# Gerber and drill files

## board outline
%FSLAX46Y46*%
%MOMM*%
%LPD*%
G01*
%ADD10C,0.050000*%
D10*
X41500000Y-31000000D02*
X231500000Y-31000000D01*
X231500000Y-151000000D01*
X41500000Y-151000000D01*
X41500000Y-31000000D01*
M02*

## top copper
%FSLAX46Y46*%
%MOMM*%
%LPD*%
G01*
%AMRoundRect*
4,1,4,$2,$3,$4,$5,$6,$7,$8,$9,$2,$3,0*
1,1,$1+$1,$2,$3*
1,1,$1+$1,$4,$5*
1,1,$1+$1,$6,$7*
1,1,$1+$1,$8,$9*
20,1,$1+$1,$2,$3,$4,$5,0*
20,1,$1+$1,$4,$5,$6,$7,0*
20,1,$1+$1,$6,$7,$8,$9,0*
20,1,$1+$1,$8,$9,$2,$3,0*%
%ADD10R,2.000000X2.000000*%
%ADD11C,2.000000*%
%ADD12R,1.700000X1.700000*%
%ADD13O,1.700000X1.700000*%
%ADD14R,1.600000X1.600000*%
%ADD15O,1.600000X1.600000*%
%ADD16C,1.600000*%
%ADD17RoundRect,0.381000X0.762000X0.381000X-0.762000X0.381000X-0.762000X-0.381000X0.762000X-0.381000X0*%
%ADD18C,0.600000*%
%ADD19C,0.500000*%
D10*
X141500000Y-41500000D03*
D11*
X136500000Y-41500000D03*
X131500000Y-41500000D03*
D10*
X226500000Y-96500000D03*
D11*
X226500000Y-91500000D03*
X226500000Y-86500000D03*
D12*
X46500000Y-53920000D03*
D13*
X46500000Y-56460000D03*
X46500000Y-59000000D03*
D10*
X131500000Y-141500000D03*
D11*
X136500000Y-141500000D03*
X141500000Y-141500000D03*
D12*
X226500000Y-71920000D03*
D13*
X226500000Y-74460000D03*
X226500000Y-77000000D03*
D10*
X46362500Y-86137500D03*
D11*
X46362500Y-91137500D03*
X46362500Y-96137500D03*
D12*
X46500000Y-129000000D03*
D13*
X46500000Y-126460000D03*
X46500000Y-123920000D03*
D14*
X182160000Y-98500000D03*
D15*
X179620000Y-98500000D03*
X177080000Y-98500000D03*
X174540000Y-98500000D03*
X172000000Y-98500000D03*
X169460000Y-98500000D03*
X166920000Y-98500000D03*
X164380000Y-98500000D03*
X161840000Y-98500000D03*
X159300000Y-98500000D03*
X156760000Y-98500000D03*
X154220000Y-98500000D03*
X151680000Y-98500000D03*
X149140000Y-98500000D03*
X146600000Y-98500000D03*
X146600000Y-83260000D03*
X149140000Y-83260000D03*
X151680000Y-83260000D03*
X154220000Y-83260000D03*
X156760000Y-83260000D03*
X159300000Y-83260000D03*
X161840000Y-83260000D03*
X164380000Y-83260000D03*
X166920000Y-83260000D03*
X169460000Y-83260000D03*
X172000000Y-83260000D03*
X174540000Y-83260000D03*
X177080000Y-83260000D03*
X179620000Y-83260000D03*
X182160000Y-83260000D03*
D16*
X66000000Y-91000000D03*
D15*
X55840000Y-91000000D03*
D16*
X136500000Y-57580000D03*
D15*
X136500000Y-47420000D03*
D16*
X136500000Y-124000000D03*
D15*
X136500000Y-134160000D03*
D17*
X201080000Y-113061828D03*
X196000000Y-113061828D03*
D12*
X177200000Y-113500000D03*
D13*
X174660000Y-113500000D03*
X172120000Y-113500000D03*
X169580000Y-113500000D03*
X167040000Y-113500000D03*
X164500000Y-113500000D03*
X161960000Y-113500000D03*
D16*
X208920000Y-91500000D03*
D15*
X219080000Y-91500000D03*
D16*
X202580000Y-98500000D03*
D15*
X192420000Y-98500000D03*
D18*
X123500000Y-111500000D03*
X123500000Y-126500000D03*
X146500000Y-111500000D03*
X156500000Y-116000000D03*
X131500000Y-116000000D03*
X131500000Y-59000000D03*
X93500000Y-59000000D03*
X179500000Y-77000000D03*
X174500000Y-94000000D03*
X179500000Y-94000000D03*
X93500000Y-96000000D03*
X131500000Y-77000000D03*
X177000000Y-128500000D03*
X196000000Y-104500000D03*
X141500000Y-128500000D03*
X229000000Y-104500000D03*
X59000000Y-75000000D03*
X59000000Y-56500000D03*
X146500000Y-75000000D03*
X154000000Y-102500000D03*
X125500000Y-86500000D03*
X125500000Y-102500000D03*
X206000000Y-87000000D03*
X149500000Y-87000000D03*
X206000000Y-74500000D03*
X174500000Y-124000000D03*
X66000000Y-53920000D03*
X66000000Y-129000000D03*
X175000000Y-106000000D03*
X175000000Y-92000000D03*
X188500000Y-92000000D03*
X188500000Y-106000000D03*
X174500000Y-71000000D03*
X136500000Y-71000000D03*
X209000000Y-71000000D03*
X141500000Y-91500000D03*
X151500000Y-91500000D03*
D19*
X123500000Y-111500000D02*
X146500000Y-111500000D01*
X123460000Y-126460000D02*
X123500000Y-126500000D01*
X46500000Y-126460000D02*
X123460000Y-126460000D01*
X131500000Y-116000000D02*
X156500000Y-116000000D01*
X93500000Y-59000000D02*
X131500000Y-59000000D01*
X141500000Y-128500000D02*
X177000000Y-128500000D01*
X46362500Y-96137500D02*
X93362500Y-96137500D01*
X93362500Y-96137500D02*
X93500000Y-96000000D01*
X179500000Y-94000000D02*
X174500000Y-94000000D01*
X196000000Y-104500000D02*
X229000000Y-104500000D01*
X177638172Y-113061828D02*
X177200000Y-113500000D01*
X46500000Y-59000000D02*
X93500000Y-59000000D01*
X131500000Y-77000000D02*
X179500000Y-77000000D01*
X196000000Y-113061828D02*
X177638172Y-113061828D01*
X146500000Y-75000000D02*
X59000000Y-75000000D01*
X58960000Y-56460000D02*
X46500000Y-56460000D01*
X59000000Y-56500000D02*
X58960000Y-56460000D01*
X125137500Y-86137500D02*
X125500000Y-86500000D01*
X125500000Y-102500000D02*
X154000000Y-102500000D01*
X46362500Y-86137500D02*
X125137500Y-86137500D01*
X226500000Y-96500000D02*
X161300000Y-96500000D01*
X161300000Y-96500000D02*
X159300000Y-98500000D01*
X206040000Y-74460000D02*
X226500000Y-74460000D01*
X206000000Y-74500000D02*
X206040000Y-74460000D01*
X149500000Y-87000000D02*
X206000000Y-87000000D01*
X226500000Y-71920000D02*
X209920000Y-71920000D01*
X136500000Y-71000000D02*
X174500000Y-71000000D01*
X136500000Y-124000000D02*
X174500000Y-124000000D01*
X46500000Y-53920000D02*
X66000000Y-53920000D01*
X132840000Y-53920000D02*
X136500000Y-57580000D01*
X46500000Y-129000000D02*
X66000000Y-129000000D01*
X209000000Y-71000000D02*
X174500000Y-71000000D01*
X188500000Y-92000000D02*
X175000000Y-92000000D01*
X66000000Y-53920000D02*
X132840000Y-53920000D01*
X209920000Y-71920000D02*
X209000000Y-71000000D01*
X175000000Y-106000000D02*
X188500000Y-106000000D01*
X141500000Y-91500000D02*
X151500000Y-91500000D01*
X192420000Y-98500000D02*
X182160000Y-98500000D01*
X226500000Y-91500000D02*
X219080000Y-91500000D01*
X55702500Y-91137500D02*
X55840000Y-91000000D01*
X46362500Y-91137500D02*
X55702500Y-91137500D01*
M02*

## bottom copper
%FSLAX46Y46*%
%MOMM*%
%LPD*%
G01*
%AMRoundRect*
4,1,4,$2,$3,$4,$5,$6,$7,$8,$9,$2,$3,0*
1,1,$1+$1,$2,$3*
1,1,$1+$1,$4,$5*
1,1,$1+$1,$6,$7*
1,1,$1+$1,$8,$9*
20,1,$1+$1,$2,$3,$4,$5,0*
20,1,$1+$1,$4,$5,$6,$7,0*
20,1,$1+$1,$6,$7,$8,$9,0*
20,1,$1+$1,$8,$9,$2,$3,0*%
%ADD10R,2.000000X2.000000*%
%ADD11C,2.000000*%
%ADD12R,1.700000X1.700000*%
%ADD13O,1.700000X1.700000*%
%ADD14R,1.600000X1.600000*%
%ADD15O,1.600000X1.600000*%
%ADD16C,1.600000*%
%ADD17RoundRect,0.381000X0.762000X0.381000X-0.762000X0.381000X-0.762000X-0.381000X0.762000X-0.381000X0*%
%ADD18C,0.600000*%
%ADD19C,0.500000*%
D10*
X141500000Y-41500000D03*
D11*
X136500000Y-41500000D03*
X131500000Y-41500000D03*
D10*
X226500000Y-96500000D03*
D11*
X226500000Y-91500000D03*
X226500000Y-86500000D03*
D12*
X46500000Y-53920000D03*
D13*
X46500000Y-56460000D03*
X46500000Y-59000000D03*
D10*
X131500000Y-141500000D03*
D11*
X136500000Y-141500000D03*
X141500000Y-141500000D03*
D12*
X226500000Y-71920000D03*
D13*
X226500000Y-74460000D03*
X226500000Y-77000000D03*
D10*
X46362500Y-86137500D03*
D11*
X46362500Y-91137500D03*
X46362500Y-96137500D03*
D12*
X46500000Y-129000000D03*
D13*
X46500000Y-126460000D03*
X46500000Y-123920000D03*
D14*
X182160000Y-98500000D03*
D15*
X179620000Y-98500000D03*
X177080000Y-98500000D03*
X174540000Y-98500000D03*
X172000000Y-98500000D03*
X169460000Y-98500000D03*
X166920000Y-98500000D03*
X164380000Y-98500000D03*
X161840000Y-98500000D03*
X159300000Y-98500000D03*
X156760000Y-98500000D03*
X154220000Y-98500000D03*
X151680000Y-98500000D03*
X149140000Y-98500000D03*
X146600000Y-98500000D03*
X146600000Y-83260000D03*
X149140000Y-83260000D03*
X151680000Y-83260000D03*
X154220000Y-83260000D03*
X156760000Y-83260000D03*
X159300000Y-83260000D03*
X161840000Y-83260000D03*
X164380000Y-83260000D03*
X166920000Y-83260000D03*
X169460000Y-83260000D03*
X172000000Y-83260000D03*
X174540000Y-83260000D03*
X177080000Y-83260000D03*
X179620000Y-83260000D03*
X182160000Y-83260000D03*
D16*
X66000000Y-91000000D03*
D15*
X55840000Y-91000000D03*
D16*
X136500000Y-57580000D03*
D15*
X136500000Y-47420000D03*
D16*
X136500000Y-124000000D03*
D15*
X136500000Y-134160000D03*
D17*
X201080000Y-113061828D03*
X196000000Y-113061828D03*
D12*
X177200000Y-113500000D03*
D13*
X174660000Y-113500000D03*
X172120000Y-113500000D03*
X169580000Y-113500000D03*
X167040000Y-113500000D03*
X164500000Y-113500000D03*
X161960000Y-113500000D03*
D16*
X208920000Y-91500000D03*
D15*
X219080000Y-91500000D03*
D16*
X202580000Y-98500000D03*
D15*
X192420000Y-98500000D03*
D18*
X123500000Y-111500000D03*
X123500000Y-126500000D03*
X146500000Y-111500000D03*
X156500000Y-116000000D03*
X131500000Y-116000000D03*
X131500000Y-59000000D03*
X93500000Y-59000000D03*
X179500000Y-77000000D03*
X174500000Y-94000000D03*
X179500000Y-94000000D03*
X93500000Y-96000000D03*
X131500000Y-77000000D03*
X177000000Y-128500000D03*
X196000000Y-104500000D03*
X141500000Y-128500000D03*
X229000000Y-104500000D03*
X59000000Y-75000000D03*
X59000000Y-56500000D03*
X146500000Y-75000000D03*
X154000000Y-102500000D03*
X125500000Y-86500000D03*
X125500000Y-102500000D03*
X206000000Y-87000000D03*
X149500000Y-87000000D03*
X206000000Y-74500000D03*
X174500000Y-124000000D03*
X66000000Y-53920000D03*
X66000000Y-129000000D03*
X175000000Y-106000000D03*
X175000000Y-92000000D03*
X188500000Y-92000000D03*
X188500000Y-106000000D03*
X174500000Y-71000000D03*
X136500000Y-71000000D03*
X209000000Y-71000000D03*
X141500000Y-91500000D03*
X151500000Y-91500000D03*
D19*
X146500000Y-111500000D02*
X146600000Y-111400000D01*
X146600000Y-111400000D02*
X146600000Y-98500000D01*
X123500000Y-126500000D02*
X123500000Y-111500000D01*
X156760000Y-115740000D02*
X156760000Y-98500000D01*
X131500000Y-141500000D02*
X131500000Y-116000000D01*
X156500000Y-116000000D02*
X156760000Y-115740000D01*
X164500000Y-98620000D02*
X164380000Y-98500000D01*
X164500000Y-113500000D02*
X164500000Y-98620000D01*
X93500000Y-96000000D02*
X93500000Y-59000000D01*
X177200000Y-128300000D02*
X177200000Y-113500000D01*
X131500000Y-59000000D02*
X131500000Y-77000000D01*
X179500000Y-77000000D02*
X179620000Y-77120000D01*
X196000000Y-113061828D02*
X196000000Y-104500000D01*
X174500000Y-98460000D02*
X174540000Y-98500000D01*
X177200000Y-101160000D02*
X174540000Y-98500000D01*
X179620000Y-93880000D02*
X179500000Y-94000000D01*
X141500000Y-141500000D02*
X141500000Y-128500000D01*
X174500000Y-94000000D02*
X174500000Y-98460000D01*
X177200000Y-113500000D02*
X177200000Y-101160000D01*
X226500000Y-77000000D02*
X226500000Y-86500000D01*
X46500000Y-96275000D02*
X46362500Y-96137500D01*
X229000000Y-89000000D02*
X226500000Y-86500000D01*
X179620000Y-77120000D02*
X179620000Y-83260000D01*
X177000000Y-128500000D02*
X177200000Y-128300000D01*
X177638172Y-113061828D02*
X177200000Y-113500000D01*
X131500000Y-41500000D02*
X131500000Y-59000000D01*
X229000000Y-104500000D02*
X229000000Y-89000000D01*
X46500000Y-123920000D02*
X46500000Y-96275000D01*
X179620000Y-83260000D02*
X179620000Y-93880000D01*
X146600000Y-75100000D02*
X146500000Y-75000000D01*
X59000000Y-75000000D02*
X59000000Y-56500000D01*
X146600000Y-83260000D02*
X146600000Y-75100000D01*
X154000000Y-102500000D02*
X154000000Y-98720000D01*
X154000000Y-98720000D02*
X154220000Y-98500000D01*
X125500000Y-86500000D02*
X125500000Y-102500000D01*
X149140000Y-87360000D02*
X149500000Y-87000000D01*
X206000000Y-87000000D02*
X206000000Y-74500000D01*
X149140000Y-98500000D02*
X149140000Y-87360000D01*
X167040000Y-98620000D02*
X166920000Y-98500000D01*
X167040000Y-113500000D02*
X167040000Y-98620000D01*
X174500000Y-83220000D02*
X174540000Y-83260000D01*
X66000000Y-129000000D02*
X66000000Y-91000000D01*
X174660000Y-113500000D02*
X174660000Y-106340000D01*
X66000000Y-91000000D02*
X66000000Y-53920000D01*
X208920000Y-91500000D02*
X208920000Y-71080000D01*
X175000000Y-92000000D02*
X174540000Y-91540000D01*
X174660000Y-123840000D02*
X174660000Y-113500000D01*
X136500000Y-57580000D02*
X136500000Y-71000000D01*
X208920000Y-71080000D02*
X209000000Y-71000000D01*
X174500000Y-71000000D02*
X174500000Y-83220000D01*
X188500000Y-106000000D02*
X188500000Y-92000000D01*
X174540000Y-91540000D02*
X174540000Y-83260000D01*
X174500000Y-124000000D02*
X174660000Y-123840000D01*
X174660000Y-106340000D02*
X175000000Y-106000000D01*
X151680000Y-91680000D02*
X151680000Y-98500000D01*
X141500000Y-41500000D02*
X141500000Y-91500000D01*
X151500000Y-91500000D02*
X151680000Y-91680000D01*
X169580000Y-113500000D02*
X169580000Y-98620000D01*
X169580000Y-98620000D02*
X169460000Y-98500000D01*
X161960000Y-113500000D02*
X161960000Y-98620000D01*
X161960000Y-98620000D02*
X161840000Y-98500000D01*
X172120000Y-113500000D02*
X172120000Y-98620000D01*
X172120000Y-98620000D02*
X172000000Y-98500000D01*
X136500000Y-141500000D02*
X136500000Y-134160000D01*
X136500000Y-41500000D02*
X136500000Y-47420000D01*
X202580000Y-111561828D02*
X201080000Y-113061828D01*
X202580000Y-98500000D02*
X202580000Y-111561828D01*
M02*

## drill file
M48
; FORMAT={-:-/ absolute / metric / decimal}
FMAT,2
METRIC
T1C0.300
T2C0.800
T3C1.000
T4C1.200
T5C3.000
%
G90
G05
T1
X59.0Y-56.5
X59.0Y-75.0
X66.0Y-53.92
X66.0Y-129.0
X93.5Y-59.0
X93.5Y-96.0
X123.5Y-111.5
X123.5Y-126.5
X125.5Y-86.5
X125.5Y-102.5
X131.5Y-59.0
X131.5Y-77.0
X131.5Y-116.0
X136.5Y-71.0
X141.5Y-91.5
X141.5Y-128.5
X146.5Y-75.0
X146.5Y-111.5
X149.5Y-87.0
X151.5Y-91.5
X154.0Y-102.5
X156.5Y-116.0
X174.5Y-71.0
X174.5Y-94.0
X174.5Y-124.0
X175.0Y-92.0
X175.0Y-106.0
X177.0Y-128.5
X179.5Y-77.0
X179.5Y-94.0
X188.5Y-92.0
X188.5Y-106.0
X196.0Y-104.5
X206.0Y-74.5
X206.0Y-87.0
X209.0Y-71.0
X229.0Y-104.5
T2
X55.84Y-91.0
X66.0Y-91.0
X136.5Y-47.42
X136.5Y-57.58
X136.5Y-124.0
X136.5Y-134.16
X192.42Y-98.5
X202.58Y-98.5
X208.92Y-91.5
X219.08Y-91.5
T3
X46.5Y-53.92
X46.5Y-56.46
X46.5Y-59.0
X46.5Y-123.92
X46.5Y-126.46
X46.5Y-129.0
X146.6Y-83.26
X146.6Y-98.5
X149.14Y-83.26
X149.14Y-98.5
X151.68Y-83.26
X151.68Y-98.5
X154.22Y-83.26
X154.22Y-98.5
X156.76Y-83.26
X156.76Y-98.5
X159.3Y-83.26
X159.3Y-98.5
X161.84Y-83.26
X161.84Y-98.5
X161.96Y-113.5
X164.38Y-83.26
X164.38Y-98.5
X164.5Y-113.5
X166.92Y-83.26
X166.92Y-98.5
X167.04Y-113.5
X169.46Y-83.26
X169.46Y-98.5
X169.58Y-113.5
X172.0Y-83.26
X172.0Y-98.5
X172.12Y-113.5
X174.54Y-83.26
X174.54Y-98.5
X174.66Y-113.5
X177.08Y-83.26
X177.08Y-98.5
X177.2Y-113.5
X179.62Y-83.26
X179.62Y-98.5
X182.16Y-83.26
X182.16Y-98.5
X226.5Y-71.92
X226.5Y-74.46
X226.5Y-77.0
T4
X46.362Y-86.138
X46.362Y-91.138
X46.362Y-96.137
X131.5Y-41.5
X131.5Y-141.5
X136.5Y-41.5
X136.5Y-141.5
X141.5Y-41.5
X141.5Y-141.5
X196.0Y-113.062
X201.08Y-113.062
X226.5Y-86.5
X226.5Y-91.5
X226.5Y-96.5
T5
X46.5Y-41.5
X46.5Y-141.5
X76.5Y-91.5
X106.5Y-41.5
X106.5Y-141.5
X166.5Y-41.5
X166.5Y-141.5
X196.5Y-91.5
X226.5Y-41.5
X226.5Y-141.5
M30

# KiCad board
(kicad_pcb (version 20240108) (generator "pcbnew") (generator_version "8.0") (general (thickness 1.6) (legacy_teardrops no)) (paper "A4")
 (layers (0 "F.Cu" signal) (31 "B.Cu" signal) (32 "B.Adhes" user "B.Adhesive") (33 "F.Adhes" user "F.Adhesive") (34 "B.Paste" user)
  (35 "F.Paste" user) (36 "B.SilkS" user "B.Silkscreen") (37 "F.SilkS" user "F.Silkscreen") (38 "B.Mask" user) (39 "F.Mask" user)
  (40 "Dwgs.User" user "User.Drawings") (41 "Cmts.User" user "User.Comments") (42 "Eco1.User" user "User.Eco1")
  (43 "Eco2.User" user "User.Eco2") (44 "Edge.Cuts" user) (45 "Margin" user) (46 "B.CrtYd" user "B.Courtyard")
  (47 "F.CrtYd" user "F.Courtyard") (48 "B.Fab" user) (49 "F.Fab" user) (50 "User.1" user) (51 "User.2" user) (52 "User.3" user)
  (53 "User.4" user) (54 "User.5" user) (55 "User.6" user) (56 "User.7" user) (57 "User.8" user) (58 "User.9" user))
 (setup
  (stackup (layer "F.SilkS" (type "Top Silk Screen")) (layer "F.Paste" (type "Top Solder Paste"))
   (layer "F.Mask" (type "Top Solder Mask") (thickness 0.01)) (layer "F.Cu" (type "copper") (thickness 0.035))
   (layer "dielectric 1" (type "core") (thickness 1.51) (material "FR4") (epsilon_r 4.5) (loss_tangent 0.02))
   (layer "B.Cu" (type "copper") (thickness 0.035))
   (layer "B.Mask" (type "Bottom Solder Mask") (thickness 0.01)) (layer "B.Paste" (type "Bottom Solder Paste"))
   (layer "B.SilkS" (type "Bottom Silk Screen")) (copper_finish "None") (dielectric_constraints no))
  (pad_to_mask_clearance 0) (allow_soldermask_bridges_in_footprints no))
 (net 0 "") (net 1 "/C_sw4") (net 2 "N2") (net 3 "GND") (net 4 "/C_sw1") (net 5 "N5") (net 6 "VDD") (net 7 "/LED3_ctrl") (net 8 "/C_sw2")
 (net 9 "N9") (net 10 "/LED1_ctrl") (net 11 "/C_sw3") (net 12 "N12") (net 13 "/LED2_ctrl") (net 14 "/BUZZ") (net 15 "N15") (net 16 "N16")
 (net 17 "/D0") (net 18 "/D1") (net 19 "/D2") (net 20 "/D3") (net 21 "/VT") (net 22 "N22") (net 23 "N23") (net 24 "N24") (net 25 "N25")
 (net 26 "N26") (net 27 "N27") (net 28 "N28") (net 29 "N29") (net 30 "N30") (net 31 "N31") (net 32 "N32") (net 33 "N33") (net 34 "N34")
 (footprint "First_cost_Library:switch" (layer "F.Cu") (at 128.5 36.5 -90)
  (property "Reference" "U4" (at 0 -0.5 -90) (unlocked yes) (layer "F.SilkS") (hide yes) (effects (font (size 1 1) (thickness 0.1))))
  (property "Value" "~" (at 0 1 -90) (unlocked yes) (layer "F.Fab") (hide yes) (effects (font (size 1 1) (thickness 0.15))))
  (pad "1" thru_hole rect (at 5 -13 270) (size 2 2) (drill 1.2) (layers "*.Cu" "*.Mask") (remove_unused_layers no) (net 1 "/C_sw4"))
  (pad "2" thru_hole circle (at 5 -8 270) (size 2 2) (drill 1.2) (layers "*.Cu" "*.Mask") (remove_unused_layers no) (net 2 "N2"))
  (pad "3" thru_hole circle (at 5 -3 270) (size 2 2) (drill 1.2) (layers "*.Cu" "*.Mask") (remove_unused_layers no) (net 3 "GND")))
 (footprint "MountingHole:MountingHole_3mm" (layer "F.Cu") (at 196.5 91.5)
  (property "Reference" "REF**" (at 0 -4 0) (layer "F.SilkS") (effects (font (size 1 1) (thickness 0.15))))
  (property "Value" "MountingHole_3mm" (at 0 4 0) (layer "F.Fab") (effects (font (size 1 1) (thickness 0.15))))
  (pad "" np_thru_hole circle (at 0 0) (size 3 3) (drill 3) (layers "*.Cu" "*.Mask")))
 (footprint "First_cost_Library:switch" (layer "F.Cu") (at 231.5 83.5 180)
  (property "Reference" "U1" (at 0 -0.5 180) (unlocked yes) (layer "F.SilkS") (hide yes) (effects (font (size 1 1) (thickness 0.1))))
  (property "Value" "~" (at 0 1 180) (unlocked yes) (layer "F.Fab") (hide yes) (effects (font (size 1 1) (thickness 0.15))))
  (pad "1" thru_hole rect (at 5 -13 180) (size 2 2) (drill 1.2) (layers "*.Cu" "*.Mask") (remove_unused_layers no) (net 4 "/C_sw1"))
  (pad "2" thru_hole circle (at 5 -8 180) (size 2 2) (drill 1.2) (layers "*.Cu" "*.Mask") (remove_unused_layers no) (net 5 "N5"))
  (pad "3" thru_hole circle (at 5 -3 180) (size 2 2) (drill 1.2) (layers "*.Cu" "*.Mask") (remove_unused_layers no) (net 3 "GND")))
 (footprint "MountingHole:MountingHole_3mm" (layer "F.Cu") (at 76.5 91.5)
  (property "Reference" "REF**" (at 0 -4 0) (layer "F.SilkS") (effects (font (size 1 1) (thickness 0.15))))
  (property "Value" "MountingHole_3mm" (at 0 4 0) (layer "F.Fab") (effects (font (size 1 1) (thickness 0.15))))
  (pad "" np_thru_hole circle (at 0 0) (size 3 3) (drill 3) (layers "*.Cu" "*.Mask")))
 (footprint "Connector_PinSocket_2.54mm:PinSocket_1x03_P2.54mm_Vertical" (layer "F.Cu") (at 46.5 53.92)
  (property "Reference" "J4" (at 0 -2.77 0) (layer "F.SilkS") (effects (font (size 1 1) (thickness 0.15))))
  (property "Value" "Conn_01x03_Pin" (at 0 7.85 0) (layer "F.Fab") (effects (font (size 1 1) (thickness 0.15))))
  (pad "1" thru_hole rect (at 0 0) (size 1.7 1.7) (drill 1) (layers "*.Cu" "*.Mask") (remove_unused_layers no) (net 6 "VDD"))
  (pad "2" thru_hole oval (at 0 2.54) (size 1.7 1.7) (drill 1) (layers "*.Cu" "*.Mask") (remove_unused_layers no) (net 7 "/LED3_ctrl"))
  (pad "3" thru_hole oval (at 0 5.08) (size 1.7 1.7) (drill 1) (layers "*.Cu" "*.Mask") (remove_unused_layers no) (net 3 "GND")))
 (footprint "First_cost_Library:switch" (layer "F.Cu") (at 144.5 146.5 90)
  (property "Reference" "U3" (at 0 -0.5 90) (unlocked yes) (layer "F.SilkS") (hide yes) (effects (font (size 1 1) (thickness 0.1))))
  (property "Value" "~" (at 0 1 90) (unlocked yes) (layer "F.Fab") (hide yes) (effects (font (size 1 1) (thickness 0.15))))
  (pad "1" thru_hole rect (at 5 -13 90) (size 2 2) (drill 1.2) (layers "*.Cu" "*.Mask") (remove_unused_layers no) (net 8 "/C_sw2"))
  (pad "2" thru_hole circle (at 5 -8 90) (size 2 2) (drill 1.2) (layers "*.Cu" "*.Mask") (remove_unused_layers no) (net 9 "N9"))
  (pad "3" thru_hole circle (at 5 -3 90) (size 2 2) (drill 1.2) (layers "*.Cu" "*.Mask") (remove_unused_layers no) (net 3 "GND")))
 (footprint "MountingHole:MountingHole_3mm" (layer "F.Cu") (at 166.5 141.5)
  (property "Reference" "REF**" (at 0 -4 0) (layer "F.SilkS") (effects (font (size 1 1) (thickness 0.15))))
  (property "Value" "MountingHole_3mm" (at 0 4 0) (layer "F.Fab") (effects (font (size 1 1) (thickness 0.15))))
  (pad "" np_thru_hole circle (at 0 0) (size 3 3) (drill 3) (layers "*.Cu" "*.Mask")))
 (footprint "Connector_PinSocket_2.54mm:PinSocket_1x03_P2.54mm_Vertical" (layer "F.Cu") (at 226.5 71.92)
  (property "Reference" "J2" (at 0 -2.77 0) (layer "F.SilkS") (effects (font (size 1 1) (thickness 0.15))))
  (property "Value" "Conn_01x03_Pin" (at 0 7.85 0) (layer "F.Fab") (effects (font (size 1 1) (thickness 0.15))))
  (pad "1" thru_hole rect (at 0 0) (size 1.7 1.7) (drill 1) (layers "*.Cu" "*.Mask") (remove_unused_layers no) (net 6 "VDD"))
  (pad "2" thru_hole oval (at 0 2.54) (size 1.7 1.7) (drill 1) (layers "*.Cu" "*.Mask") (remove_unused_layers no) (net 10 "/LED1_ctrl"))
  (pad "3" thru_hole oval (at 0 5.08) (size 1.7 1.7) (drill 1) (layers "*.Cu" "*.Mask") (remove_unused_layers no) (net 3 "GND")))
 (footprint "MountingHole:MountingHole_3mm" (layer "F.Cu") (at 106.5 141.5)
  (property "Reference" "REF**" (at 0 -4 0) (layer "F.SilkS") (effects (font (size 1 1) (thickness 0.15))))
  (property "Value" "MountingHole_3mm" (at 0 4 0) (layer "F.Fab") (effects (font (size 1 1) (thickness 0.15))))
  (pad "" np_thru_hole circle (at 0 0) (size 3 3) (drill 3) (layers "*.Cu" "*.Mask")))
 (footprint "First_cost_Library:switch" (layer "F.Cu") (at 41.3625 99.1375)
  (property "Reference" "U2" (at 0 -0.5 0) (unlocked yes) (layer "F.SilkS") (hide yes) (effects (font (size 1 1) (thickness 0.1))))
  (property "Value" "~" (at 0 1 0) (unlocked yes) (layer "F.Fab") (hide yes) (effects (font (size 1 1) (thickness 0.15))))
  (pad "1" thru_hole rect (at 5 -13) (size 2 2) (drill 1.2) (layers "*.Cu" "*.Mask") (remove_unused_layers no) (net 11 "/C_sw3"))
  (pad "2" thru_hole circle (at 5 -8) (size 2 2) (drill 1.2) (layers "*.Cu" "*.Mask") (remove_unused_layers no) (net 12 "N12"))
  (pad "3" thru_hole circle (at 5 -3) (size 2 2) (drill 1.2) (layers "*.Cu" "*.Mask") (remove_unused_layers no) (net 3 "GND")))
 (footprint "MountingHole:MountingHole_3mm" (layer "F.Cu") (at 226.5 41.5)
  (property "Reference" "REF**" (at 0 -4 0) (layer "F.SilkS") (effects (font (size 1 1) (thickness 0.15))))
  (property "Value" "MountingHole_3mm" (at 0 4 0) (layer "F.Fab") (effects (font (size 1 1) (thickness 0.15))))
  (pad "" np_thru_hole circle (at 0 0) (size 3 3) (drill 3) (layers "*.Cu" "*.Mask")))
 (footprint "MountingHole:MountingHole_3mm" (layer "F.Cu") (at 166.5 41.5)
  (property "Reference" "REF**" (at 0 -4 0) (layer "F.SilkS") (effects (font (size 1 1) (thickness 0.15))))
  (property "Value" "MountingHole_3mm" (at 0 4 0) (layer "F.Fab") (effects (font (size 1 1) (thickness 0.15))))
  (pad "" np_thru_hole circle (at 0 0) (size 3 3) (drill 3) (layers "*.Cu" "*.Mask")))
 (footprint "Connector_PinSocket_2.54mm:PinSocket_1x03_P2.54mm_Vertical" (layer "F.Cu") (at 46.5 129 180)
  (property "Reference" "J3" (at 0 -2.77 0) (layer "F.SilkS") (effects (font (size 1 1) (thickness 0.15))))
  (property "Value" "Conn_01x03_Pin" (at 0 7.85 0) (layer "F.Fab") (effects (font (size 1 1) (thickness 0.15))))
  (pad "1" thru_hole rect (at 0 0 180) (size 1.7 1.7) (drill 1) (layers "*.Cu" "*.Mask") (remove_unused_layers no) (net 6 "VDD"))
  (pad "2" thru_hole oval (at 0 2.54 180) (size 1.7 1.7) (drill 1) (layers "*.Cu" "*.Mask") (remove_unused_layers no) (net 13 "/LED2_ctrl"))
  (pad "3" thru_hole oval (at 0 5.08 180) (size 1.7 1.7) (drill 1) (layers "*.Cu" "*.Mask") (remove_unused_layers no) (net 3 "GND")))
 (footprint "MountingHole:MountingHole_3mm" (layer "F.Cu") (at 46.5 141.5)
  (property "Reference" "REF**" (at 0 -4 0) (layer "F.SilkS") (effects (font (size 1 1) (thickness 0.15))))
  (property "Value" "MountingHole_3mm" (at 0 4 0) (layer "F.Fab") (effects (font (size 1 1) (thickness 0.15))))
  (pad "" np_thru_hole circle (at 0 0) (size 3 3) (drill 3) (layers "*.Cu" "*.Mask")))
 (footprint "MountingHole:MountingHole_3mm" (layer "F.Cu") (at 46.5 41.5)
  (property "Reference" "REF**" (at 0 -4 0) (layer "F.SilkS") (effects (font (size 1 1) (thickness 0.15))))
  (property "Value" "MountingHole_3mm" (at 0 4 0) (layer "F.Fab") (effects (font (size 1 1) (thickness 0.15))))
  (pad "" np_thru_hole circle (at 0 0) (size 3 3) (drill 3) (layers "*.Cu" "*.Mask")))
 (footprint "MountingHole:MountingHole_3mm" (layer "F.Cu") (at 226.5 141.5)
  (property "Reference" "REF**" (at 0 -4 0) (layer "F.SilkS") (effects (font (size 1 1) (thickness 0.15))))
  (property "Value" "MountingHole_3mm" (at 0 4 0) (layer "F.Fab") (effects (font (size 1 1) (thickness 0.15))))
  (pad "" np_thru_hole circle (at 0 0) (size 3 3) (drill 3) (layers "*.Cu" "*.Mask")))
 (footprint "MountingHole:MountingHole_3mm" (layer "F.Cu") (at 106.5 41.5)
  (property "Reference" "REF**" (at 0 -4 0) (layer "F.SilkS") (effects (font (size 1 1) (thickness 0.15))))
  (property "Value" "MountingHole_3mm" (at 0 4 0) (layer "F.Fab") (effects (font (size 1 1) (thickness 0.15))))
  (pad "" np_thru_hole circle (at 0 0) (size 3 3) (drill 3) (layers "*.Cu" "*.Mask")))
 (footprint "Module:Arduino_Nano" (layer "B.Cu") (at 182.16 98.5 90)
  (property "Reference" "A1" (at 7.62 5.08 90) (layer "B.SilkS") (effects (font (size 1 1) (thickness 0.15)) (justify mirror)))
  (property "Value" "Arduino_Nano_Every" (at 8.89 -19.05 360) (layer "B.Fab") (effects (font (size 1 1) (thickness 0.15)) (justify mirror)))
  (pad "1" thru_hole rect (at 0 0 90) (size 1.6 1.6) (drill 1) (layers "*.Cu" "*.Mask") (remove_unused_layers no) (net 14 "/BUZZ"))
  (pad "2" thru_hole oval (at 0 -2.54 90) (size 1.6 1.6) (drill 1) (layers "*.Cu" "*.Mask") (remove_unused_layers no) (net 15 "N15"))
  (pad "3" thru_hole oval (at 0 -5.08 90) (size 1.6 1.6) (drill 1) (layers "*.Cu" "*.Mask") (remove_unused_layers no) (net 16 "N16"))
  (pad "4" thru_hole oval (at 0 -7.62 90) (size 1.6 1.6) (drill 1) (layers "*.Cu" "*.Mask") (remove_unused_layers no) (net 3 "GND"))
  (pad "5" thru_hole oval (at 0 -10.16 90) (size 1.6 1.6) (drill 1) (layers "*.Cu" "*.Mask") (remove_unused_layers no) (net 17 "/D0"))
  (pad "6" thru_hole oval (at 0 -12.7 90) (size 1.6 1.6) (drill 1) (layers "*.Cu" "*.Mask") (remove_unused_layers no) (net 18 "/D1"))
  (pad "7" thru_hole oval (at 0 -15.24 90) (size 1.6 1.6) (drill 1) (layers "*.Cu" "*.Mask") (remove_unused_layers no) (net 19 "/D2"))
  (pad "8" thru_hole oval (at 0 -17.78 90) (size 1.6 1.6) (drill 1) (layers "*.Cu" "*.Mask") (remove_unused_layers no) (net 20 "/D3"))
  (pad "9" thru_hole oval (at 0 -20.32 90) (size 1.6 1.6) (drill 1) (layers "*.Cu" "*.Mask") (remove_unused_layers no) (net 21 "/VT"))
  (pad "10" thru_hole oval (at 0 -22.86 90) (size 1.6 1.6) (drill 1) (layers "*.Cu" "*.Mask") (remove_unused_layers no) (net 4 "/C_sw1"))
  (pad "11" thru_hole oval (at 0 -25.4 90) (size 1.6 1.6) (drill 1) (layers "*.Cu" "*.Mask") (remove_unused_layers no) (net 8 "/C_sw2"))
  (pad "12" thru_hole oval (at 0 -27.94 90) (size 1.6 1.6) (drill 1) (layers "*.Cu" "*.Mask") (remove_unused_layers no) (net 11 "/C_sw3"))
  (pad "13" thru_hole oval (at 0 -30.48 90) (size 1.6 1.6) (drill 1) (layers "*.Cu" "*.Mask") (remove_unused_layers no) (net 1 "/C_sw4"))
  (pad "14" thru_hole oval (at 0 -33.02 90) (size 1.6 1.6) (drill 1) (layers "*.Cu" "*.Mask") (remove_unused_layers no)
   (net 10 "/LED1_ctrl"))
  (pad "15" thru_hole oval (at 0 -35.56 90) (size 1.6 1.6) (drill 1) (layers "*.Cu" "*.Mask") (remove_unused_layers no)
   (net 13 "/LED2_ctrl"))
  (pad "16" thru_hole oval (at 15.24 -35.56 90) (size 1.6 1.6) (drill 1) (layers "*.Cu" "*.Mask") (remove_unused_layers no)
   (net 7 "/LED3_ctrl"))
  (pad "17" thru_hole oval (at 15.24 -33.02 90) (size 1.6 1.6) (drill 1) (layers "*.Cu" "*.Mask") (remove_unused_layers no) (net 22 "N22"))
  (pad "18" thru_hole oval (at 15.24 -30.48 90) (size 1.6 1.6) (drill 1) (layers "*.Cu" "*.Mask") (remove_unused_layers no) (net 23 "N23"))
  (pad "19" thru_hole oval (at 15.24 -27.94 90) (size 1.6 1.6) (drill 1) (layers "*.Cu" "*.Mask") (remove_unused_layers no) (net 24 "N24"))
  (pad "20" thru_hole oval (at 15.24 -25.4 90) (size 1.6 1.6) (drill 1) (layers "*.Cu" "*.Mask") (remove_unused_layers no) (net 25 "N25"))
  (pad "21" thru_hole oval (at 15.24 -22.86 90) (size 1.6 1.6) (drill 1) (layers "*.Cu" "*.Mask") (remove_unused_layers no) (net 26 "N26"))
  (pad "22" thru_hole oval (at 15.24 -20.32 90) (size 1.6 1.6) (drill 1) (layers "*.Cu" "*.Mask") (remove_unused_layers no) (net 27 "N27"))
  (pad "23" thru_hole oval (at 15.24 -17.78 90) (size 1.6 1.6) (drill 1) (layers "*.Cu" "*.Mask") (remove_unused_layers no) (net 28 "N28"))
  (pad "24" thru_hole oval (at 15.24 -15.24 90) (size 1.6 1.6) (drill 1) (layers "*.Cu" "*.Mask") (remove_unused_layers no) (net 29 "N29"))
  (pad "25" thru_hole oval (at 15.24 -12.7 90) (size 1.6 1.6) (drill 1) (layers "*.Cu" "*.Mask") (remove_unused_layers no) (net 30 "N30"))
  (pad "26" thru_hole oval (at 15.24 -10.16 90) (size 1.6 1.6) (drill 1) (layers "*.Cu" "*.Mask") (remove_unused_layers no) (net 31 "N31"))
  (pad "27" thru_hole oval (at 15.24 -7.62 90) (size 1.6 1.6) (drill 1) (layers "*.Cu" "*.Mask") (remove_unused_layers no) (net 6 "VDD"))
  (pad "28" thru_hole oval (at 15.24 -5.08 90) (size 1.6 1.6) (drill 1) (layers "*.Cu" "*.Mask") (remove_unused_layers no) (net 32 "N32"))
  (pad "29" thru_hole oval (at 15.24 -2.54 90) (size 1.6 1.6) (drill 1) (layers "*.Cu" "*.Mask") (remove_unused_layers no) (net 3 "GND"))
  (pad "30" thru_hole oval (at 15.24 0 90) (size 1.6 1.6) (drill 1) (layers "*.Cu" "*.Mask") (remove_unused_layers no) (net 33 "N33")))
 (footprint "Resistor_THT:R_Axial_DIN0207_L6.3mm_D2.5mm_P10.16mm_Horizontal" (layer "B.Cu") (at 66 91 180)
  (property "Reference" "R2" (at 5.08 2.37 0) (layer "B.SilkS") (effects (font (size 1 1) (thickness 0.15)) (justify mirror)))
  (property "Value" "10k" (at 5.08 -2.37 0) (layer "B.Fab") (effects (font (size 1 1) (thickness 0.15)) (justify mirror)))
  (pad "1" thru_hole circle (at 0 0 180) (size 1.6 1.6) (drill 0.8) (layers "*.Cu" "*.Mask") (remove_unused_layers no) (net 6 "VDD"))
  (pad "2" thru_hole oval (at 10.16 0 180) (size 1.6 1.6) (drill 0.8) (layers "*.Cu" "*.Mask") (remove_unused_layers no) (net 12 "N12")))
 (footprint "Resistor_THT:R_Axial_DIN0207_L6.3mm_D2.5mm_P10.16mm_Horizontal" (layer "B.Cu") (at 136.5 57.58 90)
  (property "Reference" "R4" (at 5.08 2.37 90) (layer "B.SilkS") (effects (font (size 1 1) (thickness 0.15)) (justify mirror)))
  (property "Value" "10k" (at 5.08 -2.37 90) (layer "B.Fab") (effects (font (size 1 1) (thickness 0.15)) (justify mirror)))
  (pad "1" thru_hole circle (at 0 0 90) (size 1.6 1.6) (drill 0.8) (layers "*.Cu" "*.Mask") (remove_unused_layers no) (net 6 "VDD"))
  (pad "2" thru_hole oval (at 10.16 0 90) (size 1.6 1.6) (drill 0.8) (layers "*.Cu" "*.Mask") (remove_unused_layers no) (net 2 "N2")))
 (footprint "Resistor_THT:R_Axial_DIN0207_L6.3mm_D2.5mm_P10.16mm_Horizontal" (layer "B.Cu") (at 136.5 124 -90)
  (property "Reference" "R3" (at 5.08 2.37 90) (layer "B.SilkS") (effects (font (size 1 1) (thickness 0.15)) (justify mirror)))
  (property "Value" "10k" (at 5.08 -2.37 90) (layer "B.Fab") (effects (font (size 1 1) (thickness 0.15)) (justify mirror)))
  (pad "1" thru_hole circle (at 0 0 270) (size 1.6 1.6) (drill 0.8) (layers "*.Cu" "*.Mask") (remove_unused_layers no) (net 6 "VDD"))
  (pad "2" thru_hole oval (at 10.16 0 270) (size 1.6 1.6) (drill 0.8) (layers "*.Cu" "*.Mask") (remove_unused_layers no) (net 9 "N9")))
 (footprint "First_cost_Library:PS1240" (layer "B.Cu") (at 198.54 102.901828 180)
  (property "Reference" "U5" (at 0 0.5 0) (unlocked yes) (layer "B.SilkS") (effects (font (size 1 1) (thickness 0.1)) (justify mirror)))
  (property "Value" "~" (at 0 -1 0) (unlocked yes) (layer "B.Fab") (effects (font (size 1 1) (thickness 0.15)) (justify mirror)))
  (pad "1" thru_hole roundrect (at -2.54 -10.16 180) (size 2.286 1.524) (drill 1.2) (layers "*.Cu" "*.Mask") (remove_unused_layers no)
   (roundrect_rratio 0.25) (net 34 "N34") (thermal_bridge_angle 45))
  (pad "2" thru_hole roundrect (at 2.54 -10.16 180) (size 2.286 1.524) (drill 1.2) (layers "*.Cu" "*.Mask") (remove_unused_layers no)
   (roundrect_rratio 0.25) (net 3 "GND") (thermal_bridge_angle 45)))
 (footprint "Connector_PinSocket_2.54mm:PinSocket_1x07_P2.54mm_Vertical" (layer "B.Cu") (at 177.2 113.5 90)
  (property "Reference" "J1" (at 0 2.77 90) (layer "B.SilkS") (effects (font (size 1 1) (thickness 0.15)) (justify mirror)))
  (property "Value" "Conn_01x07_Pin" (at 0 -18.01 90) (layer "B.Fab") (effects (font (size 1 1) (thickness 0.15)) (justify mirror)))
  (pad "1" thru_hole rect (at 0 0 90) (size 1.7 1.7) (drill 1) (layers "*.Cu" "*.Mask") (remove_unused_layers no) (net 3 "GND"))
  (pad "2" thru_hole oval (at 0 -2.54 90) (size 1.7 1.7) (drill 1) (layers "*.Cu" "*.Mask") (remove_unused_layers no) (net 6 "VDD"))
  (pad "3" thru_hole oval (at 0 -5.08 90) (size 1.7 1.7) (drill 1) (layers "*.Cu" "*.Mask") (remove_unused_layers no) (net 17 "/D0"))
  (pad "4" thru_hole oval (at 0 -7.62 90) (size 1.7 1.7) (drill 1) (layers "*.Cu" "*.Mask") (remove_unused_layers no) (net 18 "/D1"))
  (pad "5" thru_hole oval (at 0 -10.16 90) (size 1.7 1.7) (drill 1) (layers "*.Cu" "*.Mask") (remove_unused_layers no) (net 19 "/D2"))
  (pad "6" thru_hole oval (at 0 -12.7 90) (size 1.7 1.7) (drill 1) (layers "*.Cu" "*.Mask") (remove_unused_layers no) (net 20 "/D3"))
  (pad "7" thru_hole oval (at 0 -15.24 90) (size 1.7 1.7) (drill 1) (layers "*.Cu" "*.Mask") (remove_unused_layers no) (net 21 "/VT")))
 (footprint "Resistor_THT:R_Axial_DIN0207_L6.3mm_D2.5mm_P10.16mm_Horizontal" (layer "B.Cu") (at 208.92 91.5)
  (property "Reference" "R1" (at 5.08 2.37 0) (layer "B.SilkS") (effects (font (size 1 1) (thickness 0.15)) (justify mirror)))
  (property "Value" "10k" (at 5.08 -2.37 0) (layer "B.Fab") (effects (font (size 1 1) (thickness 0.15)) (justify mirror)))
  (pad "1" thru_hole circle (at 0 0) (size 1.6 1.6) (drill 0.8) (layers "*.Cu" "*.Mask") (remove_unused_layers no) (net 6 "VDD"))
  (pad "2" thru_hole oval (at 10.16 0) (size 1.6 1.6) (drill 0.8) (layers "*.Cu" "*.Mask") (remove_unused_layers no) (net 5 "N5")))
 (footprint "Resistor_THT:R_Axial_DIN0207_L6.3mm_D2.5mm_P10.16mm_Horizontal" (layer "B.Cu") (at 202.58 98.5 180)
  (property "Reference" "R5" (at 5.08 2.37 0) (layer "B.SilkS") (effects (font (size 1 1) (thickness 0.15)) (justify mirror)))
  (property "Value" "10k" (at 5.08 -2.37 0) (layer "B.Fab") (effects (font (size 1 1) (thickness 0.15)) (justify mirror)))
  (pad "1" thru_hole circle (at 0 0 180) (size 1.6 1.6) (drill 0.8) (layers "*.Cu" "*.Mask") (remove_unused_layers no) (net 34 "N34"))
  (pad "2" thru_hole oval (at 10.16 0 180) (size 1.6 1.6) (drill 0.8) (layers "*.Cu" "*.Mask") (remove_unused_layers no) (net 14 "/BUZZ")))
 (gr_rect (start 41.5 31) (end 231.5 151) (stroke (width 0.05) (type default)) (fill none) (layer "Edge.Cuts"))
 (segment (start 123.5 111.5) (end 146.5 111.5) (width 0.5) (layer "F.Cu") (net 13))
 (segment (start 123.46 126.46) (end 123.5 126.5) (width 0.5) (layer "F.Cu") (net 13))
 (segment (start 46.5 126.46) (end 123.46 126.46) (width 0.5) (layer "F.Cu") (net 13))
 (via (at 123.5 111.5) (size 0.6) (drill 0.3) (layers "F.Cu" "B.Cu") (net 13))
 (via (at 123.5 126.5) (size 0.6) (drill 0.3) (layers "F.Cu" "B.Cu") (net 13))
 (via (at 146.5 111.5) (size 0.6) (drill 0.3) (layers "F.Cu" "B.Cu") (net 13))
 (segment (start 146.5 111.5) (end 146.6 111.4) (width 0.5) (layer "B.Cu") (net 13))
 (segment (start 146.6 111.4) (end 146.6 98.5) (width 0.5) (layer "B.Cu") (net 13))
 (segment (start 123.5 126.5) (end 123.5 111.5) (width 0.5) (layer "B.Cu") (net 13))
 (segment (start 131.5 116) (end 156.5 116) (width 0.5) (layer "F.Cu") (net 8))
 (via (at 156.5 116) (size 0.6) (drill 0.3) (layers "F.Cu" "B.Cu") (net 8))
 (via (at 131.5 116) (size 0.6) (drill 0.3) (layers "F.Cu" "B.Cu") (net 8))
 (segment (start 156.76 115.74) (end 156.76 98.5) (width 0.5) (layer "B.Cu") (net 8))
 (segment (start 131.5 141.5) (end 131.5 116) (width 0.5) (layer "B.Cu") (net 8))
 (segment (start 156.5 116) (end 156.76 115.74) (width 0.5) (layer "B.Cu") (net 8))
 (segment (start 164.5 98.62) (end 164.38 98.5) (width 0.5) (layer "B.Cu") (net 20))
 (segment (start 164.5 113.5) (end 164.5 98.62) (width 0.5) (layer "B.Cu") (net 20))
 (segment (start 93.5 59) (end 131.5 59) (width 0.5) (layer "F.Cu") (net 3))
 (segment (start 141.5 128.5) (end 177 128.5) (width 0.5) (layer "F.Cu") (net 3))
 (segment (start 46.3625 96.1375) (end 93.3625 96.1375) (width 0.5) (layer "F.Cu") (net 3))
 (segment (start 93.3625 96.1375) (end 93.5 96) (width 0.5) (layer "F.Cu") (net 3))
 (segment (start 179.5 94) (end 174.5 94) (width 0.5) (layer "F.Cu") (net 3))
 (segment (start 196 104.5) (end 229 104.5) (width 0.5) (layer "F.Cu") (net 3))
 (segment (start 177.638172 113.061828) (end 177.2 113.5) (width 0.5) (layer "F.Cu") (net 3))
 (segment (start 46.5 59) (end 93.5 59) (width 0.5) (layer "F.Cu") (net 3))
 (segment (start 131.5 77) (end 179.5 77) (width 0.5) (layer "F.Cu") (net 3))
 (segment (start 196 113.061828) (end 177.638172 113.061828) (width 0.5) (layer "F.Cu") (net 3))
 (via (at 131.5 59) (size 0.6) (drill 0.3) (layers "F.Cu" "B.Cu") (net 3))
 (via (at 93.5 59) (size 0.6) (drill 0.3) (layers "F.Cu" "B.Cu") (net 3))
 (via (at 179.5 77) (size 0.6) (drill 0.3) (layers "F.Cu" "B.Cu") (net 3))
 (via (at 174.5 94) (size 0.6) (drill 0.3) (layers "F.Cu" "B.Cu") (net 3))
 (via (at 179.5 94) (size 0.6) (drill 0.3) (layers "F.Cu" "B.Cu") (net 3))
 (via (at 93.5 96) (size 0.6) (drill 0.3) (layers "F.Cu" "B.Cu") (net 3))
 (via (at 131.5 77) (size 0.6) (drill 0.3) (layers "F.Cu" "B.Cu") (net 3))
 (via (at 177 128.5) (size 0.6) (drill 0.3) (layers "F.Cu" "B.Cu") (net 3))
 (via (at 196 104.5) (size 0.6) (drill 0.3) (layers "F.Cu" "B.Cu") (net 3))
 (via (at 141.5 128.5) (size 0.6) (drill 0.3) (layers "F.Cu" "B.Cu") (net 3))
 (via (at 229 104.5) (size 0.6) (drill 0.3) (layers "F.Cu" "B.Cu") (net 3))
 (segment (start 93.5 96) (end 93.5 59) (width 0.5) (layer "B.Cu") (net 3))
 (segment (start 177.2 128.3) (end 177.2 113.5) (width 0.5) (layer "B.Cu") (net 3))
 (segment (start 131.5 59) (end 131.5 77) (width 0.5) (layer "B.Cu") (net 3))
 (segment (start 179.5 77) (end 179.62 77.12) (width 0.5) (layer "B.Cu") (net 3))
 (segment (start 196 113.061828) (end 196 104.5) (width 0.5) (layer "B.Cu") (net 3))
 (segment (start 174.5 98.46) (end 174.54 98.5) (width 0.5) (layer "B.Cu") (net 3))
 (segment (start 177.2 101.16) (end 174.54 98.5) (width 0.5) (layer "B.Cu") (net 3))
 (segment (start 179.62 93.88) (end 179.5 94) (width 0.5) (layer "B.Cu") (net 3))
 (segment (start 141.5 141.5) (end 141.5 128.5) (width 0.5) (layer "B.Cu") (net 3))
 (segment (start 174.5 94) (end 174.5 98.46) (width 0.5) (layer "B.Cu") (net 3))
 (segment (start 177.2 113.5) (end 177.2 101.16) (width 0.5) (layer "B.Cu") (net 3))
 (segment (start 226.5 77) (end 226.5 86.5) (width 0.5) (layer "B.Cu") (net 3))
 (segment (start 46.5 96.275) (end 46.3625 96.1375) (width 0.5) (layer "B.Cu") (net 3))
 (segment (start 229 89) (end 226.5 86.5) (width 0.5) (layer "B.Cu") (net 3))
 (segment (start 179.62 77.12) (end 179.62 83.26) (width 0.5) (layer "B.Cu") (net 3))
 (segment (start 177 128.5) (end 177.2 128.3) (width 0.5) (layer "B.Cu") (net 3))
 (segment (start 177.638172 113.061828) (end 177.2 113.5) (width 0.5) (layer "B.Cu") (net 3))
 (segment (start 131.5 41.5) (end 131.5 59) (width 0.5) (layer "B.Cu") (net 3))
 (segment (start 229 104.5) (end 229 89) (width 0.5) (layer "B.Cu") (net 3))
 (segment (start 46.5 123.92) (end 46.5 96.275) (width 0.5) (layer "B.Cu") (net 3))
 (segment (start 179.62 83.26) (end 179.62 93.88) (width 0.5) (layer "B.Cu") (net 3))
 (segment (start 146.5 75) (end 59 75) (width 0.5) (layer "F.Cu") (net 7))
 (segment (start 58.96 56.46) (end 46.5 56.46) (width 0.5) (layer "F.Cu") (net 7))
 (segment (start 59 56.5) (end 58.96 56.46) (width 0.5) (layer "F.Cu") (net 7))
 (via (at 59 75) (size 0.6) (drill 0.3) (layers "F.Cu" "B.Cu") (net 7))
 (via (at 59 56.5) (size 0.6) (drill 0.3) (layers "F.Cu" "B.Cu") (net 7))
 (via (at 146.5 75) (size 0.6) (drill 0.3) (layers "F.Cu" "B.Cu") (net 7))
 (segment (start 146.6 75.1) (end 146.5 75) (width 0.5) (layer "B.Cu") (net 7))
 (segment (start 59 75) (end 59 56.5) (width 0.5) (layer "B.Cu") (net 7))
 (segment (start 146.6 83.26) (end 146.6 75.1) (width 0.5) (layer "B.Cu") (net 7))
 (segment (start 125.1375 86.1375) (end 125.5 86.5) (width 0.5) (layer "F.Cu") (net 11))
 (segment (start 125.5 102.5) (end 154 102.5) (width 0.5) (layer "F.Cu") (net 11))
 (segment (start 46.3625 86.1375) (end 125.1375 86.1375) (width 0.5) (layer "F.Cu") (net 11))
 (via (at 154 102.5) (size 0.6) (drill 0.3) (layers "F.Cu" "B.Cu") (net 11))
 (via (at 125.5 86.5) (size 0.6) (drill 0.3) (layers "F.Cu" "B.Cu") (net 11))
 (via (at 125.5 102.5) (size 0.6) (drill 0.3) (layers "F.Cu" "B.Cu") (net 11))
 (segment (start 154 102.5) (end 154 98.72) (width 0.5) (layer "B.Cu") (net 11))
 (segment (start 154 98.72) (end 154.22 98.5) (width 0.5) (layer "B.Cu") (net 11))
 (segment (start 125.5 86.5) (end 125.5 102.5) (width 0.5) (layer "B.Cu") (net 11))
 (segment (start 226.5 96.5) (end 161.3 96.5) (width 0.5) (layer "F.Cu") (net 4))
 (segment (start 161.3 96.5) (end 159.3 98.5) (width 0.5) (layer "F.Cu") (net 4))
 (segment (start 206.04 74.46) (end 226.5 74.46) (width 0.5) (layer "F.Cu") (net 10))
 (segment (start 206 74.5) (end 206.04 74.46) (width 0.5) (layer "F.Cu") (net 10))
 (segment (start 149.5 87) (end 206 87) (width 0.5) (layer "F.Cu") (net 10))
 (via (at 206 87) (size 0.6) (drill 0.3) (layers "F.Cu" "B.Cu") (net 10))
 (via (at 149.5 87) (size 0.6) (drill 0.3) (layers "F.Cu" "B.Cu") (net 10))
 (via (at 206 74.5) (size 0.6) (drill 0.3) (layers "F.Cu" "B.Cu") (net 10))
 (segment (start 149.14 87.36) (end 149.5 87) (width 0.5) (layer "B.Cu") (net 10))
 (segment (start 206 87) (end 206 74.5) (width 0.5) (layer "B.Cu") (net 10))
 (segment (start 149.14 98.5) (end 149.14 87.36) (width 0.5) (layer "B.Cu") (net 10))
 (segment (start 167.04 98.62) (end 166.92 98.5) (width 0.5) (layer "B.Cu") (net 19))
 (segment (start 167.04 113.5) (end 167.04 98.62) (width 0.5) (layer "B.Cu") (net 19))
 (segment (start 226.5 71.92) (end 209.92 71.92) (width 0.5) (layer "F.Cu") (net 6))
 (segment (start 136.5 71) (end 174.5 71) (width 0.5) (layer "F.Cu") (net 6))
 (segment (start 136.5 124) (end 174.5 124) (width 0.5) (layer "F.Cu") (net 6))
 (segment (start 46.5 53.92) (end 66 53.92) (width 0.5) (layer "F.Cu") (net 6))
 (segment (start 132.84 53.92) (end 136.5 57.58) (width 0.5) (layer "F.Cu") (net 6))
 (segment (start 46.5 129) (end 66 129) (width 0.5) (layer "F.Cu") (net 6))
 (segment (start 209 71) (end 174.5 71) (width 0.5) (layer "F.Cu") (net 6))
 (segment (start 188.5 92) (end 175 92) (width 0.5) (layer "F.Cu") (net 6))
 (segment (start 66 53.92) (end 132.84 53.92) (width 0.5) (layer "F.Cu") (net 6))
 (segment (start 209.92 71.92) (end 209 71) (width 0.5) (layer "F.Cu") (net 6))
 (segment (start 175 106) (end 188.5 106) (width 0.5) (layer "F.Cu") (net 6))
 (via (at 174.5 124) (size 0.6) (drill 0.3) (layers "F.Cu" "B.Cu") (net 6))
 (via (at 66 53.92) (size 0.6) (drill 0.3) (layers "F.Cu" "B.Cu") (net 6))
 (via (at 66 129) (size 0.6) (drill 0.3) (layers "F.Cu" "B.Cu") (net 6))
 (via (at 175 106) (size 0.6) (drill 0.3) (layers "F.Cu" "B.Cu") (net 6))
 (via (at 175 92) (size 0.6) (drill 0.3) (layers "F.Cu" "B.Cu") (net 6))
 (via (at 188.5 92) (size 0.6) (drill 0.3) (layers "F.Cu" "B.Cu") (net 6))
 (via (at 188.5 106) (size 0.6) (drill 0.3) (layers "F.Cu" "B.Cu") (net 6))
 (via (at 174.5 71) (size 0.6) (drill 0.3) (layers "F.Cu" "B.Cu") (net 6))
 (via (at 136.5 71) (size 0.6) (drill 0.3) (layers "F.Cu" "B.Cu") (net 6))
 (via (at 209 71) (size 0.6) (drill 0.3) (layers "F.Cu" "B.Cu") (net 6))
 (segment (start 174.5 83.22) (end 174.54 83.26) (width 0.5) (layer "B.Cu") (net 6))
 (segment (start 66 129) (end 66 91) (width 0.5) (layer "B.Cu") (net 6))
 (segment (start 174.66 113.5) (end 174.66 106.34) (width 0.5) (layer "B.Cu") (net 6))
 (segment (start 66 91) (end 66 53.92) (width 0.5) (layer "B.Cu") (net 6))
 (segment (start 208.92 91.5) (end 208.92 71.08) (width 0.5) (layer "B.Cu") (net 6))
 (segment (start 175 92) (end 174.54 91.54) (width 0.5) (layer "B.Cu") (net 6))
 (segment (start 174.66 123.84) (end 174.66 113.5) (width 0.5) (layer "B.Cu") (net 6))
 (segment (start 136.5 57.58) (end 136.5 71) (width 0.5) (layer "B.Cu") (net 6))
 (segment (start 208.92 71.08) (end 209 71) (width 0.5) (layer "B.Cu") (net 6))
 (segment (start 174.5 71) (end 174.5 83.22) (width 0.5) (layer "B.Cu") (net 6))
 (segment (start 188.5 106) (end 188.5 92) (width 0.5) (layer "B.Cu") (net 6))
 (segment (start 174.54 91.54) (end 174.54 83.26) (width 0.5) (layer "B.Cu") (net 6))
 (segment (start 174.5 124) (end 174.66 123.84) (width 0.5) (layer "B.Cu") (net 6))
 (segment (start 174.66 106.34) (end 175 106) (width 0.5) (layer "B.Cu") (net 6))
 (segment (start 141.5 91.5) (end 151.5 91.5) (width 0.5) (layer "F.Cu") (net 1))
 (via (at 141.5 91.5) (size 0.6) (drill 0.3) (layers "F.Cu" "B.Cu") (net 1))
 (via (at 151.5 91.5) (size 0.6) (drill 0.3) (layers "F.Cu" "B.Cu") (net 1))
 (segment (start 151.68 91.68) (end 151.68 98.5) (width 0.5) (layer "B.Cu") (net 1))
 (segment (start 141.5 41.5) (end 141.5 91.5) (width 0.5) (layer "B.Cu") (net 1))
 (segment (start 151.5 91.5) (end 151.68 91.68) (width 0.5) (layer "B.Cu") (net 1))
 (segment (start 169.58 113.5) (end 169.58 98.62) (width 0.5) (layer "B.Cu") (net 18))
 (segment (start 169.58 98.62) (end 169.46 98.5) (width 0.5) (layer "B.Cu") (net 18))
 (segment (start 161.96 113.5) (end 161.96 98.62) (width 0.5) (layer "B.Cu") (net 21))
 (segment (start 161.96 98.62) (end 161.84 98.5) (width 0.5) (layer "B.Cu") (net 21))
 (segment (start 172.12 113.5) (end 172.12 98.62) (width 0.5) (layer "B.Cu") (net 17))
 (segment (start 172.12 98.62) (end 172 98.5) (width 0.5) (layer "B.Cu") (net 17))
 (segment (start 192.42 98.5) (end 182.16 98.5) (width 0.5) (layer "F.Cu") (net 14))
 (segment (start 226.5 91.5) (end 219.08 91.5) (width 0.5) (layer "F.Cu") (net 5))
 (segment (start 55.7025 91.1375) (end 55.84 91) (width 0.5) (layer "F.Cu") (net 12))
 (segment (start 46.3625 91.1375) (end 55.7025 91.1375) (width 0.5) (layer "F.Cu") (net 12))
 (segment (start 136.5 141.5) (end 136.5 134.16) (width 0.5) (layer "B.Cu") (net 9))
 (segment (start 136.5 41.5) (end 136.5 47.42) (width 0.5) (layer "B.Cu") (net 2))
 (segment (start 202.58 111.561828) (end 201.08 113.061828) (width 0.5) (layer "B.Cu") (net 34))
 (segment (start 202.58 98.5) (end 202.58 111.561828) (width 0.5) (layer "B.Cu") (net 34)))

